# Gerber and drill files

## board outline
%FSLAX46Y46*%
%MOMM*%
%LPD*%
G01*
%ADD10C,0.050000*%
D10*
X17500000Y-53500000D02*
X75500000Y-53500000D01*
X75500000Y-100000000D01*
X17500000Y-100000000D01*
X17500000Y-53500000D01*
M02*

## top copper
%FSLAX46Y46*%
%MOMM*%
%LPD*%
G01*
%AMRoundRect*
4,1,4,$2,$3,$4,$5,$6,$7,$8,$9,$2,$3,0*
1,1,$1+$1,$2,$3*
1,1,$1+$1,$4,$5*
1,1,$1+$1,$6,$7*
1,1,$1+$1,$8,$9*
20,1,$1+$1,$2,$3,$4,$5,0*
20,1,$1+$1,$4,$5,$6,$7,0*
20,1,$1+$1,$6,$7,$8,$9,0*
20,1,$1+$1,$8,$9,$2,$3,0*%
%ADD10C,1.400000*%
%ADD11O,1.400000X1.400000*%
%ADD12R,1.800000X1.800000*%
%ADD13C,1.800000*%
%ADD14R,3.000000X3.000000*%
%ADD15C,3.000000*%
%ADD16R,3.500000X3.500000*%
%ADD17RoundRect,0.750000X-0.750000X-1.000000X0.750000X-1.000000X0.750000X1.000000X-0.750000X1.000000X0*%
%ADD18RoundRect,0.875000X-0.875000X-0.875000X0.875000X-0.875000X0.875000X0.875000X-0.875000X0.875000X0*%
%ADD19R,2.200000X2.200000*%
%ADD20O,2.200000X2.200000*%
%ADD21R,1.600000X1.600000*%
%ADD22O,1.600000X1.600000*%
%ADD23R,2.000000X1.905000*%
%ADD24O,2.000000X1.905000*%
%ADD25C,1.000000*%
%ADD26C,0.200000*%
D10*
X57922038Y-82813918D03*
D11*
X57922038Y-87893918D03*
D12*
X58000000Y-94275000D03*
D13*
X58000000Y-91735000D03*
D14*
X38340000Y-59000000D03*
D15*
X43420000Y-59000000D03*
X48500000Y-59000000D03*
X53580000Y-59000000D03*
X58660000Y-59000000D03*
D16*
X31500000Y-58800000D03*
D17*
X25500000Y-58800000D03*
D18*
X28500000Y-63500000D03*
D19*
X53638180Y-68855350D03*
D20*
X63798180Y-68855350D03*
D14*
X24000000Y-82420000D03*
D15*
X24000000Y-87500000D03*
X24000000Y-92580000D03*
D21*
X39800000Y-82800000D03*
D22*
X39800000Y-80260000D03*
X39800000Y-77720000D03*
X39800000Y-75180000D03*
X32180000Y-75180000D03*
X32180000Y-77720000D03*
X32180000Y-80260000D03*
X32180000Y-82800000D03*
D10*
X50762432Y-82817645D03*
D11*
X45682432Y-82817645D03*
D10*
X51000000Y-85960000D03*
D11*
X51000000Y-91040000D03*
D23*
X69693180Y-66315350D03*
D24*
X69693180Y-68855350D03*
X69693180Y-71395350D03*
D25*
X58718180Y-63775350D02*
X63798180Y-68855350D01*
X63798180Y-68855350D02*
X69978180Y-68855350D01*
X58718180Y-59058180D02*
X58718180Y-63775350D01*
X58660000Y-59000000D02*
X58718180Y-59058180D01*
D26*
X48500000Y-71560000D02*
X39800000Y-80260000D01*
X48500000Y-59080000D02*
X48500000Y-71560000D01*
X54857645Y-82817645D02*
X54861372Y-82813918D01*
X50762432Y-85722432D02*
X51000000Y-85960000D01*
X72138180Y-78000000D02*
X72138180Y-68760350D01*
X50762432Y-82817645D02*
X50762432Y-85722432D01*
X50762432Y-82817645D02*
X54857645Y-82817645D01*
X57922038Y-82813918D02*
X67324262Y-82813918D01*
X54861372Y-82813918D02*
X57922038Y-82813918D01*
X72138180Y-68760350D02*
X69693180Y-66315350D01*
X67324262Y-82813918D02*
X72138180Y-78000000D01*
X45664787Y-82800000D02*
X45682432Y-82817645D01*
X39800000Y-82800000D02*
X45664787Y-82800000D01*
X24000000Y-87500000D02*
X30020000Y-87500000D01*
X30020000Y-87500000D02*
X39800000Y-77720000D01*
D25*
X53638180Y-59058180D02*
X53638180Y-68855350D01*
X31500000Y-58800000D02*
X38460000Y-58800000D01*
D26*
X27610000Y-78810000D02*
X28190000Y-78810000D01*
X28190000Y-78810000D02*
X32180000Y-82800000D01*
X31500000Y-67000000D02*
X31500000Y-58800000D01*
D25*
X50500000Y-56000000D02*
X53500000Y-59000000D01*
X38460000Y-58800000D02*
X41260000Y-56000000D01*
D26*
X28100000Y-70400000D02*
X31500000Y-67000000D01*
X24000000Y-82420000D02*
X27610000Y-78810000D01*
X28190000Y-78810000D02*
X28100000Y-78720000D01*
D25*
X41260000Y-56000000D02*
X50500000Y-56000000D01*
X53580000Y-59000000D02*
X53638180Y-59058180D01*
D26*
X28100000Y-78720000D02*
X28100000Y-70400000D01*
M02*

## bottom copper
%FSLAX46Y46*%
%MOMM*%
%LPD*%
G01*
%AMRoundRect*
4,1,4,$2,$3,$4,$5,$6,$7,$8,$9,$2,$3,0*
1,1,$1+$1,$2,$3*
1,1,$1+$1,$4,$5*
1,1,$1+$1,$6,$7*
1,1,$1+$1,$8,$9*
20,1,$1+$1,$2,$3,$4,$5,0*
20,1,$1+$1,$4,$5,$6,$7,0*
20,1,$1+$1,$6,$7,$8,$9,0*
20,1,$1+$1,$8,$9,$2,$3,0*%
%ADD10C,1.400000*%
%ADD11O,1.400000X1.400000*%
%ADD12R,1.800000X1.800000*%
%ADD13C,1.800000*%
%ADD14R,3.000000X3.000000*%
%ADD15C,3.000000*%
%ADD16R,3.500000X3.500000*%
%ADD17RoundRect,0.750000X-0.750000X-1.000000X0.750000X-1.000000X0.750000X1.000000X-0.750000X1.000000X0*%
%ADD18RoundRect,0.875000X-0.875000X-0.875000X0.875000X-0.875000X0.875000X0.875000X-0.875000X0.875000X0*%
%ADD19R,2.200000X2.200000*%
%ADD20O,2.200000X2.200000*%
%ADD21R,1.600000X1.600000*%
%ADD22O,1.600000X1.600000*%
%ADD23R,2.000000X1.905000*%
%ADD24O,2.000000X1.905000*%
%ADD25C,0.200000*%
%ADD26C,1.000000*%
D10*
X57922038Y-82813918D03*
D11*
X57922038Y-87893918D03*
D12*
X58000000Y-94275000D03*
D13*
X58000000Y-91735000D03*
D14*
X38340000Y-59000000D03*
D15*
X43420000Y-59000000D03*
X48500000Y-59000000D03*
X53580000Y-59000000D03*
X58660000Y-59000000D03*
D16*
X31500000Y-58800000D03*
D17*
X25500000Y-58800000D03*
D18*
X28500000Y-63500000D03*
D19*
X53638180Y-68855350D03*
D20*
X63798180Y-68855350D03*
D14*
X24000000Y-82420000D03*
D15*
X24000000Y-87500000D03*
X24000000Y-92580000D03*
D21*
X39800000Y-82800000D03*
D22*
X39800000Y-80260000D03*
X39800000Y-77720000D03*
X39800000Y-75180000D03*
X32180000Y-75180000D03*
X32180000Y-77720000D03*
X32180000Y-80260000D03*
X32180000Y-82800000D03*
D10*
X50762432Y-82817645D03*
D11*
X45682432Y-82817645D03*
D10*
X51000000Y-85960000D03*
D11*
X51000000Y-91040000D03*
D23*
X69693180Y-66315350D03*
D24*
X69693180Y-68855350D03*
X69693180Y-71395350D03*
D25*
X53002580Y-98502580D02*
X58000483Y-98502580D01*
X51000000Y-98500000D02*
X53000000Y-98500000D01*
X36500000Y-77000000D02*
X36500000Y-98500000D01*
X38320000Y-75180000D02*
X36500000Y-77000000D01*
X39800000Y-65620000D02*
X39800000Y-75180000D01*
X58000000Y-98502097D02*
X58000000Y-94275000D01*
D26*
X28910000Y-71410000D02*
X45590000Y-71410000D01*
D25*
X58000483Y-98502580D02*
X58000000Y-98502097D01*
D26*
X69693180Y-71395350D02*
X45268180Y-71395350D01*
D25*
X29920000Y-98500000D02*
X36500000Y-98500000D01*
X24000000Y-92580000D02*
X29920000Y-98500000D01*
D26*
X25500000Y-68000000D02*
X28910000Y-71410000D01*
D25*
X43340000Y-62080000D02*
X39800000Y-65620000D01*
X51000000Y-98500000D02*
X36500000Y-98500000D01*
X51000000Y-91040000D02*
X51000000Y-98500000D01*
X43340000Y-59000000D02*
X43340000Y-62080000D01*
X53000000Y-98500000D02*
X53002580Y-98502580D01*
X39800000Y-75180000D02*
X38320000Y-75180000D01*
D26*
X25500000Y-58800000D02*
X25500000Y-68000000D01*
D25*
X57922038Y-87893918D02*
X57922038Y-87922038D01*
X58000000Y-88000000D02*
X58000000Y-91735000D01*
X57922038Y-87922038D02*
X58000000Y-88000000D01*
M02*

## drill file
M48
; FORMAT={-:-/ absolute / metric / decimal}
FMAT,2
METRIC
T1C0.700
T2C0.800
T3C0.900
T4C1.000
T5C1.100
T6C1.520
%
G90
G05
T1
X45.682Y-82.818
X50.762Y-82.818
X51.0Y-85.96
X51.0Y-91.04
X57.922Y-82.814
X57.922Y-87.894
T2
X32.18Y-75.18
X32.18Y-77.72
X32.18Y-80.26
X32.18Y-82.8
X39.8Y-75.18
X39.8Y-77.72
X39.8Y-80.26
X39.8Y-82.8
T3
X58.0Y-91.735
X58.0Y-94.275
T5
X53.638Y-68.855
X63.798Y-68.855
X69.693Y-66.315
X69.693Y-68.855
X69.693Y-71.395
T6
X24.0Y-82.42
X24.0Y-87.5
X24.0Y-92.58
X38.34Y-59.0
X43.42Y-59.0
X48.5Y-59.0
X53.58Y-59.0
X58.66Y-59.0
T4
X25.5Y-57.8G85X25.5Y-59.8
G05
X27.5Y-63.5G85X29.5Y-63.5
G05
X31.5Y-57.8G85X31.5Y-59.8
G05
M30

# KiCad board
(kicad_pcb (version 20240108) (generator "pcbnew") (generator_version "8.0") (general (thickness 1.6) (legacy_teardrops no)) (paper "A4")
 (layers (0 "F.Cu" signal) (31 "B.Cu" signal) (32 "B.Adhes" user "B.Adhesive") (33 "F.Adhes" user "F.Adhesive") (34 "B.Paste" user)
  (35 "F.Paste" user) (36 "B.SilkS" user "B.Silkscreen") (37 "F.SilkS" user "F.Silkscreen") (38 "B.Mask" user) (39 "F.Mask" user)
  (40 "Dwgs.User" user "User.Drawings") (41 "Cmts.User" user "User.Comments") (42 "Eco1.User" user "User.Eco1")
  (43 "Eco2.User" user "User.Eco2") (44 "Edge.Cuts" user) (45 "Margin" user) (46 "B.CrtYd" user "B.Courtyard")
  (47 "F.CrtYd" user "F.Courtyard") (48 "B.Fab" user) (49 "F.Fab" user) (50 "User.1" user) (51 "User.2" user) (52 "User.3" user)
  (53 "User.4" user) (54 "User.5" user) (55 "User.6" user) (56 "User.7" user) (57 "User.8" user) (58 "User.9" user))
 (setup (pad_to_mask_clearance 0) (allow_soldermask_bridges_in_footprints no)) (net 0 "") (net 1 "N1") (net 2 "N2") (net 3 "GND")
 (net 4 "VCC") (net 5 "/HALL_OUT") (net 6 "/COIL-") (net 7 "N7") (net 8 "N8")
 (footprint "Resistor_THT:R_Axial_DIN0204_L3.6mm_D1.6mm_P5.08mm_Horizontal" (layer "F.Cu") (at 57.922038 82.813918 -90)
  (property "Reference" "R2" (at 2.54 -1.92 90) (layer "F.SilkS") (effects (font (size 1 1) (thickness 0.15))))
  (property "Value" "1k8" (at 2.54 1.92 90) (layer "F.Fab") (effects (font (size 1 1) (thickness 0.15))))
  (pad "1" thru_hole circle (at 0 0 270) (size 1.4 1.4) (drill 0.7) (layers "*.Cu" "*.Mask") (remove_unused_layers no) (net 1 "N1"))
  (pad "2" thru_hole oval (at 5.08 0 270) (size 1.4 1.4) (drill 0.7) (layers "*.Cu" "*.Mask") (remove_unused_layers no) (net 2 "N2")))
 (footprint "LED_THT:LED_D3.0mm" (layer "F.Cu") (at 58 94.275 90)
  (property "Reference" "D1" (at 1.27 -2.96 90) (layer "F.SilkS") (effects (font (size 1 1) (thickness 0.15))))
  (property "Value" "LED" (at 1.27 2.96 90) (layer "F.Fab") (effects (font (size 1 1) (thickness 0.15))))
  (pad "1" thru_hole rect (at 0 0 90) (size 1.8 1.8) (drill 0.9) (layers "*.Cu" "*.Mask") (remove_unused_layers no) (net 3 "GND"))
  (pad "2" thru_hole circle (at 2.54 0 90) (size 1.8 1.8) (drill 0.9) (layers "*.Cu" "*.Mask") (remove_unused_layers no) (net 2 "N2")))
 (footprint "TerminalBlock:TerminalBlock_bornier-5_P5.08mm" (layer "F.Cu") (at 38.34 59)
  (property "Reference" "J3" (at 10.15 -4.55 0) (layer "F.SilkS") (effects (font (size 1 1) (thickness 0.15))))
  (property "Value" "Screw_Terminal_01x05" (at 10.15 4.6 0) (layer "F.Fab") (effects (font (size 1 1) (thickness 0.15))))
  (pad "1" thru_hole rect (at 0 0) (size 3 3) (drill 1.52) (layers "*.Cu" "*.Mask") (remove_unused_layers no) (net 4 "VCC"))
  (pad "2" thru_hole circle (at 5.08 0) (size 3 3) (drill 1.52) (layers "*.Cu" "*.Mask") (remove_unused_layers no) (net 3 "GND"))
  (pad "3" thru_hole circle (at 10.16 0) (size 3 3) (drill 1.52) (layers "*.Cu" "*.Mask") (remove_unused_layers no) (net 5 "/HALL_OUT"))
  (pad "4" thru_hole circle (at 15.24 0) (size 3 3) (drill 1.52) (layers "*.Cu" "*.Mask") (remove_unused_layers no) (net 4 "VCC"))
  (pad "5" thru_hole circle (at 20.32 0) (size 3 3) (drill 1.52) (layers "*.Cu" "*.Mask") (remove_unused_layers no) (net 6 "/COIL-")))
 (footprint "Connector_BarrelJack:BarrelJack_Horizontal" (layer "F.Cu") (at 31.5 58.8)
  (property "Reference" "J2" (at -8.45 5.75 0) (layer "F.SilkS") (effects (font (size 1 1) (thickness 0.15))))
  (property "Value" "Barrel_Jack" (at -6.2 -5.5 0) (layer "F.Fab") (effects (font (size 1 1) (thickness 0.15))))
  (pad "1" thru_hole rect (at 0 0) (size 3.5 3.5) (drill oval 1 3) (layers "*.Cu" "*.Mask") (remove_unused_layers no) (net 4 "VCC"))
  (pad "2" thru_hole roundrect (at -6 0) (size 3 3.5) (drill oval 1 3) (layers "*.Cu" "*.Mask") (remove_unused_layers no)
   (roundrect_rratio 0.25) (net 3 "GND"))
  (pad "3" thru_hole roundrect (at -3 4.7) (size 3.5 3.5) (drill oval 3 1) (layers "*.Cu" "*.Mask") (remove_unused_layers no)
   (roundrect_rratio 0.25)))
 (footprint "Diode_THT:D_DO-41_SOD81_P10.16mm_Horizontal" (layer "F.Cu") (at 53.63818 68.85535)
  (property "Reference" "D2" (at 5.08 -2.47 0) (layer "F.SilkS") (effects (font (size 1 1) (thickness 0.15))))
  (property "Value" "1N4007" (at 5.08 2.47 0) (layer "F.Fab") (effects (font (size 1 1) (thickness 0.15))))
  (pad "1" thru_hole rect (at 0 0) (size 2.2 2.2) (drill 1.1) (layers "*.Cu" "*.Mask") (remove_unused_layers no) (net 4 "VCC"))
  (pad "2" thru_hole oval (at 10.16 0) (size 2.2 2.2) (drill 1.1) (layers "*.Cu" "*.Mask") (remove_unused_layers no) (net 6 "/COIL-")))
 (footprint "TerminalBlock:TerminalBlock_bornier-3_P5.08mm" (layer "F.Cu") (at 24 82.42 -90)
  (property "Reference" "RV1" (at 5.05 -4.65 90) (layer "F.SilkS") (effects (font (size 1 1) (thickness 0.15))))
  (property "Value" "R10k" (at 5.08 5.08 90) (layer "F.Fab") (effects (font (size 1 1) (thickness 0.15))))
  (pad "1" thru_hole rect (at 0 0 270) (size 3 3) (drill 1.52) (layers "*.Cu" "*.Mask") (remove_unused_layers no) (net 4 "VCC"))
  (pad "2" thru_hole circle (at 5.08 0 270) (size 3 3) (drill 1.52) (layers "*.Cu" "*.Mask") (remove_unused_layers no) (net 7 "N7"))
  (pad "3" thru_hole circle (at 10.16 0 270) (size 3 3) (drill 1.52) (layers "*.Cu" "*.Mask") (remove_unused_layers no) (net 3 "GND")))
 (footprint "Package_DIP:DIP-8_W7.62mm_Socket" (layer "F.Cu") (at 39.8 82.8 180)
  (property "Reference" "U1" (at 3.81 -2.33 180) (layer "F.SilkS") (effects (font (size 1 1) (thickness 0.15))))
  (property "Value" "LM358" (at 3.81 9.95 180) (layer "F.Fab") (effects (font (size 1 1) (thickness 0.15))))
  (pad "1" thru_hole rect (at 0 0 180) (size 1.6 1.6) (drill 0.8) (layers "*.Cu" "*.Mask") (remove_unused_layers no) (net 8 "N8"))
  (pad "2" thru_hole oval (at 0 2.54 180) (size 1.6 1.6) (drill 0.8) (layers "*.Cu" "*.Mask") (remove_unused_layers no) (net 5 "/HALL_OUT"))
  (pad "3" thru_hole oval (at 0 5.08 180) (size 1.6 1.6) (drill 0.8) (layers "*.Cu" "*.Mask") (remove_unused_layers no) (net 7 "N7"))
  (pad "4" thru_hole oval (at 0 7.62 180) (size 1.6 1.6) (drill 0.8) (layers "*.Cu" "*.Mask") (remove_unused_layers no) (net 3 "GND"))
  (pad "5" thru_hole oval (at 7.62 7.62 180) (size 1.6 1.6) (drill 0.8) (layers "*.Cu" "*.Mask") (remove_unused_layers no))
  (pad "6" thru_hole oval (at 7.62 5.08 180) (size 1.6 1.6) (drill 0.8) (layers "*.Cu" "*.Mask") (remove_unused_layers no))
  (pad "7" thru_hole oval (at 7.62 2.54 180) (size 1.6 1.6) (drill 0.8) (layers "*.Cu" "*.Mask") (remove_unused_layers no))
  (pad "8" thru_hole oval (at 7.62 0 180) (size 1.6 1.6) (drill 0.8) (layers "*.Cu" "*.Mask") (remove_unused_layers no) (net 4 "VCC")))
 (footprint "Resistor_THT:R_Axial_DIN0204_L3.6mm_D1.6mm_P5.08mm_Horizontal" (layer "F.Cu") (at 50.762432 82.817645 180)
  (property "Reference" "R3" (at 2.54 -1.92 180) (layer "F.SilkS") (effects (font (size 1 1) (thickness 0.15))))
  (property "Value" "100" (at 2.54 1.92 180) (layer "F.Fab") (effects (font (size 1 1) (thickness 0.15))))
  (pad "1" thru_hole circle (at 0 0 180) (size 1.4 1.4) (drill 0.7) (layers "*.Cu" "*.Mask") (remove_unused_layers no) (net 1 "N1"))
  (pad "2" thru_hole oval (at 5.08 0 180) (size 1.4 1.4) (drill 0.7) (layers "*.Cu" "*.Mask") (remove_unused_layers no) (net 8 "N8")))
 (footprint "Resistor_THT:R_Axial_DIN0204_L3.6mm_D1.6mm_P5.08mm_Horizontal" (layer "F.Cu") (at 51 85.96 -90)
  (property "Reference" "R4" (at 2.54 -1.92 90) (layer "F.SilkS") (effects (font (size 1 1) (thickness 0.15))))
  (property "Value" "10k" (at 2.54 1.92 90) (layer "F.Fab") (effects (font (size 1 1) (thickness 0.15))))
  (pad "1" thru_hole circle (at 0 0 270) (size 1.4 1.4) (drill 0.7) (layers "*.Cu" "*.Mask") (remove_unused_layers no) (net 1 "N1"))
  (pad "2" thru_hole oval (at 5.08 0 270) (size 1.4 1.4) (drill 0.7) (layers "*.Cu" "*.Mask") (remove_unused_layers no) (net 3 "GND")))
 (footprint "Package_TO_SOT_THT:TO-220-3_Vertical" (layer "F.Cu") (at 69.69318 66.31535 -90)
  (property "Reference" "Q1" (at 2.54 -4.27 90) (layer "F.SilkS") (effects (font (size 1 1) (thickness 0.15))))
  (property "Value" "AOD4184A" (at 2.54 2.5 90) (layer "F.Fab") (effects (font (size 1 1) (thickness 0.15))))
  (pad "1" thru_hole rect (at 0 0 270) (size 1.905 2) (drill 1.1) (layers "*.Cu" "*.Mask") (remove_unused_layers no) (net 1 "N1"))
  (pad "2" thru_hole oval (at 2.54 0 270) (size 1.905 2) (drill 1.1) (layers "*.Cu" "*.Mask") (remove_unused_layers no) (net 6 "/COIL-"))
  (pad "3" thru_hole oval (at 5.08 0 270) (size 1.905 2) (drill 1.1) (layers "*.Cu" "*.Mask") (remove_unused_layers no) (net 3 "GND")))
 (gr_rect (start 17.5 53.5) (end 75.5 100) (stroke (width 0.05) (type default)) (fill none) (layer "Edge.Cuts"))
 (segment (start 58.71818 63.77535) (end 63.79818 68.85535) (width 1) (layer "F.Cu") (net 6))
 (segment (start 63.79818 68.85535) (end 69.97818 68.85535) (width 1) (layer "F.Cu") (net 6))
 (segment (start 58.71818 59.05818) (end 58.71818 63.77535) (width 1) (layer "F.Cu") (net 6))
 (segment (start 58.66 59) (end 58.71818 59.05818) (width 1) (layer "F.Cu") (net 6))
 (segment (start 53.00258 98.50258) (end 58.000483 98.50258) (width 0.2) (layer "B.Cu") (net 3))
 (segment (start 51 98.5) (end 53 98.5) (width 0.2) (layer "B.Cu") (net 3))
 (segment (start 36.5 77) (end 36.5 98.5) (width 0.2) (layer "B.Cu") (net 3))
 (segment (start 38.32 75.18) (end 36.5 77) (width 0.2) (layer "B.Cu") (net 3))
 (segment (start 39.8 65.62) (end 39.8 75.18) (width 0.2) (layer "B.Cu") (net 3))
 (segment (start 58 98.502097) (end 58 94.275) (width 0.2) (layer "B.Cu") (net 3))
 (segment (start 28.91 71.41) (end 45.59 71.41) (width 1) (layer "B.Cu") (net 3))
 (segment (start 58.000483 98.50258) (end 58 98.502097) (width 0.2) (layer "B.Cu") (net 3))
 (segment (start 69.69318 71.39535) (end 45.26818 71.39535) (width 1) (layer "B.Cu") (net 3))
 (segment (start 29.92 98.5) (end 36.5 98.5) (width 0.2) (layer "B.Cu") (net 3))
 (segment (start 24 92.58) (end 29.92 98.5) (width 0.2) (layer "B.Cu") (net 3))
 (segment (start 25.5 68) (end 28.91 71.41) (width 1) (layer "B.Cu") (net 3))
 (segment (start 43.34 62.08) (end 39.8 65.62) (width 0.2) (layer "B.Cu") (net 3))
 (segment (start 51 98.5) (end 36.5 98.5) (width 0.2) (layer "B.Cu") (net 3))
 (segment (start 51 91.04) (end 51 98.5) (width 0.2) (layer "B.Cu") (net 3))
 (segment (start 43.34 59) (end 43.34 62.08) (width 0.2) (layer "B.Cu") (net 3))
 (segment (start 53 98.5) (end 53.00258 98.50258) (width 0.2) (layer "B.Cu") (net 3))
 (segment (start 39.8 75.18) (end 38.32 75.18) (width 0.2) (layer "B.Cu") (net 3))
 (segment (start 25.5 58.8) (end 25.5 68) (width 1) (layer "B.Cu") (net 3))
 (segment (start 48.5 71.56) (end 39.8 80.26) (width 0.2) (layer "F.Cu") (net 5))
 (segment (start 48.5 59.08) (end 48.5 71.56) (width 0.2) (layer "F.Cu") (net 5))
 (segment (start 54.857645 82.817645) (end 54.861372 82.813918) (width 0.2) (layer "F.Cu") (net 1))
 (segment (start 50.762432 85.722432) (end 51 85.96) (width 0.2) (layer "F.Cu") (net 1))
 (segment (start 72.13818 78) (end 72.13818 68.76035) (width 0.2) (layer "F.Cu") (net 1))
 (segment (start 50.762432 82.817645) (end 50.762432 85.722432) (width 0.2) (layer "F.Cu") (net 1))
 (segment (start 50.762432 82.817645) (end 54.857645 82.817645) (width 0.2) (layer "F.Cu") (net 1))
 (segment (start 57.922038 82.813918) (end 67.324262 82.813918) (width 0.2) (layer "F.Cu") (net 1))
 (segment (start 54.861372 82.813918) (end 57.922038 82.813918) (width 0.2) (layer "F.Cu") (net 1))
 (segment (start 72.13818 68.76035) (end 69.69318 66.31535) (width 0.2) (layer "F.Cu") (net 1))
 (segment (start 67.324262 82.813918) (end 72.13818 78) (width 0.2) (layer "F.Cu") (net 1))
 (segment (start 45.664787 82.8) (end 45.682432 82.817645) (width 0.2) (layer "F.Cu") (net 8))
 (segment (start 39.8 82.8) (end 45.664787 82.8) (width 0.2) (layer "F.Cu") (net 8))
 (segment (start 57.922038 87.893918) (end 57.922038 87.922038) (width 0.2) (layer "B.Cu") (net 2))
 (segment (start 58 88) (end 58 91.735) (width 0.2) (layer "B.Cu") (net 2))
 (segment (start 57.922038 87.922038) (end 58 88) (width 0.2) (layer "B.Cu") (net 2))
 (segment (start 24 87.5) (end 30.02 87.5) (width 0.2) (layer "F.Cu") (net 7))
 (segment (start 30.02 87.5) (end 39.8 77.72) (width 0.2) (layer "F.Cu") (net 7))
 (segment (start 53.63818 59.05818) (end 53.63818 68.85535) (width 1) (layer "F.Cu") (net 4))
 (segment (start 31.5 58.8) (end 38.46 58.8) (width 1) (layer "F.Cu") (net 4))
 (segment (start 27.61 78.81) (end 28.19 78.81) (width 0.2) (layer "F.Cu") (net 4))
 (segment (start 28.19 78.81) (end 32.18 82.8) (width 0.2) (layer "F.Cu") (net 4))
 (segment (start 31.5 67) (end 31.5 58.8) (width 0.2) (layer "F.Cu") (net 4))
 (segment (start 50.5 56) (end 53.5 59) (width 1) (layer "F.Cu") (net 4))
 (segment (start 38.46 58.8) (end 41.26 56) (width 1) (layer "F.Cu") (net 4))
 (segment (start 28.1 70.4) (end 31.5 67) (width 0.2) (layer "F.Cu") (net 4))
 (segment (start 24 82.42) (end 27.61 78.81) (width 0.2) (layer "F.Cu") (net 4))
 (segment (start 28.19 78.81) (end 28.1 78.72) (width 0.2) (layer "F.Cu") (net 4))
 (segment (start 41.26 56) (end 50.5 56) (width 1) (layer "F.Cu") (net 4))
 (segment (start 53.58 59) (end 53.63818 59.05818) (width 1) (layer "F.Cu") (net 4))
 (segment (start 28.1 78.72) (end 28.1 70.4) (width 0.2) (layer "F.Cu") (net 4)))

